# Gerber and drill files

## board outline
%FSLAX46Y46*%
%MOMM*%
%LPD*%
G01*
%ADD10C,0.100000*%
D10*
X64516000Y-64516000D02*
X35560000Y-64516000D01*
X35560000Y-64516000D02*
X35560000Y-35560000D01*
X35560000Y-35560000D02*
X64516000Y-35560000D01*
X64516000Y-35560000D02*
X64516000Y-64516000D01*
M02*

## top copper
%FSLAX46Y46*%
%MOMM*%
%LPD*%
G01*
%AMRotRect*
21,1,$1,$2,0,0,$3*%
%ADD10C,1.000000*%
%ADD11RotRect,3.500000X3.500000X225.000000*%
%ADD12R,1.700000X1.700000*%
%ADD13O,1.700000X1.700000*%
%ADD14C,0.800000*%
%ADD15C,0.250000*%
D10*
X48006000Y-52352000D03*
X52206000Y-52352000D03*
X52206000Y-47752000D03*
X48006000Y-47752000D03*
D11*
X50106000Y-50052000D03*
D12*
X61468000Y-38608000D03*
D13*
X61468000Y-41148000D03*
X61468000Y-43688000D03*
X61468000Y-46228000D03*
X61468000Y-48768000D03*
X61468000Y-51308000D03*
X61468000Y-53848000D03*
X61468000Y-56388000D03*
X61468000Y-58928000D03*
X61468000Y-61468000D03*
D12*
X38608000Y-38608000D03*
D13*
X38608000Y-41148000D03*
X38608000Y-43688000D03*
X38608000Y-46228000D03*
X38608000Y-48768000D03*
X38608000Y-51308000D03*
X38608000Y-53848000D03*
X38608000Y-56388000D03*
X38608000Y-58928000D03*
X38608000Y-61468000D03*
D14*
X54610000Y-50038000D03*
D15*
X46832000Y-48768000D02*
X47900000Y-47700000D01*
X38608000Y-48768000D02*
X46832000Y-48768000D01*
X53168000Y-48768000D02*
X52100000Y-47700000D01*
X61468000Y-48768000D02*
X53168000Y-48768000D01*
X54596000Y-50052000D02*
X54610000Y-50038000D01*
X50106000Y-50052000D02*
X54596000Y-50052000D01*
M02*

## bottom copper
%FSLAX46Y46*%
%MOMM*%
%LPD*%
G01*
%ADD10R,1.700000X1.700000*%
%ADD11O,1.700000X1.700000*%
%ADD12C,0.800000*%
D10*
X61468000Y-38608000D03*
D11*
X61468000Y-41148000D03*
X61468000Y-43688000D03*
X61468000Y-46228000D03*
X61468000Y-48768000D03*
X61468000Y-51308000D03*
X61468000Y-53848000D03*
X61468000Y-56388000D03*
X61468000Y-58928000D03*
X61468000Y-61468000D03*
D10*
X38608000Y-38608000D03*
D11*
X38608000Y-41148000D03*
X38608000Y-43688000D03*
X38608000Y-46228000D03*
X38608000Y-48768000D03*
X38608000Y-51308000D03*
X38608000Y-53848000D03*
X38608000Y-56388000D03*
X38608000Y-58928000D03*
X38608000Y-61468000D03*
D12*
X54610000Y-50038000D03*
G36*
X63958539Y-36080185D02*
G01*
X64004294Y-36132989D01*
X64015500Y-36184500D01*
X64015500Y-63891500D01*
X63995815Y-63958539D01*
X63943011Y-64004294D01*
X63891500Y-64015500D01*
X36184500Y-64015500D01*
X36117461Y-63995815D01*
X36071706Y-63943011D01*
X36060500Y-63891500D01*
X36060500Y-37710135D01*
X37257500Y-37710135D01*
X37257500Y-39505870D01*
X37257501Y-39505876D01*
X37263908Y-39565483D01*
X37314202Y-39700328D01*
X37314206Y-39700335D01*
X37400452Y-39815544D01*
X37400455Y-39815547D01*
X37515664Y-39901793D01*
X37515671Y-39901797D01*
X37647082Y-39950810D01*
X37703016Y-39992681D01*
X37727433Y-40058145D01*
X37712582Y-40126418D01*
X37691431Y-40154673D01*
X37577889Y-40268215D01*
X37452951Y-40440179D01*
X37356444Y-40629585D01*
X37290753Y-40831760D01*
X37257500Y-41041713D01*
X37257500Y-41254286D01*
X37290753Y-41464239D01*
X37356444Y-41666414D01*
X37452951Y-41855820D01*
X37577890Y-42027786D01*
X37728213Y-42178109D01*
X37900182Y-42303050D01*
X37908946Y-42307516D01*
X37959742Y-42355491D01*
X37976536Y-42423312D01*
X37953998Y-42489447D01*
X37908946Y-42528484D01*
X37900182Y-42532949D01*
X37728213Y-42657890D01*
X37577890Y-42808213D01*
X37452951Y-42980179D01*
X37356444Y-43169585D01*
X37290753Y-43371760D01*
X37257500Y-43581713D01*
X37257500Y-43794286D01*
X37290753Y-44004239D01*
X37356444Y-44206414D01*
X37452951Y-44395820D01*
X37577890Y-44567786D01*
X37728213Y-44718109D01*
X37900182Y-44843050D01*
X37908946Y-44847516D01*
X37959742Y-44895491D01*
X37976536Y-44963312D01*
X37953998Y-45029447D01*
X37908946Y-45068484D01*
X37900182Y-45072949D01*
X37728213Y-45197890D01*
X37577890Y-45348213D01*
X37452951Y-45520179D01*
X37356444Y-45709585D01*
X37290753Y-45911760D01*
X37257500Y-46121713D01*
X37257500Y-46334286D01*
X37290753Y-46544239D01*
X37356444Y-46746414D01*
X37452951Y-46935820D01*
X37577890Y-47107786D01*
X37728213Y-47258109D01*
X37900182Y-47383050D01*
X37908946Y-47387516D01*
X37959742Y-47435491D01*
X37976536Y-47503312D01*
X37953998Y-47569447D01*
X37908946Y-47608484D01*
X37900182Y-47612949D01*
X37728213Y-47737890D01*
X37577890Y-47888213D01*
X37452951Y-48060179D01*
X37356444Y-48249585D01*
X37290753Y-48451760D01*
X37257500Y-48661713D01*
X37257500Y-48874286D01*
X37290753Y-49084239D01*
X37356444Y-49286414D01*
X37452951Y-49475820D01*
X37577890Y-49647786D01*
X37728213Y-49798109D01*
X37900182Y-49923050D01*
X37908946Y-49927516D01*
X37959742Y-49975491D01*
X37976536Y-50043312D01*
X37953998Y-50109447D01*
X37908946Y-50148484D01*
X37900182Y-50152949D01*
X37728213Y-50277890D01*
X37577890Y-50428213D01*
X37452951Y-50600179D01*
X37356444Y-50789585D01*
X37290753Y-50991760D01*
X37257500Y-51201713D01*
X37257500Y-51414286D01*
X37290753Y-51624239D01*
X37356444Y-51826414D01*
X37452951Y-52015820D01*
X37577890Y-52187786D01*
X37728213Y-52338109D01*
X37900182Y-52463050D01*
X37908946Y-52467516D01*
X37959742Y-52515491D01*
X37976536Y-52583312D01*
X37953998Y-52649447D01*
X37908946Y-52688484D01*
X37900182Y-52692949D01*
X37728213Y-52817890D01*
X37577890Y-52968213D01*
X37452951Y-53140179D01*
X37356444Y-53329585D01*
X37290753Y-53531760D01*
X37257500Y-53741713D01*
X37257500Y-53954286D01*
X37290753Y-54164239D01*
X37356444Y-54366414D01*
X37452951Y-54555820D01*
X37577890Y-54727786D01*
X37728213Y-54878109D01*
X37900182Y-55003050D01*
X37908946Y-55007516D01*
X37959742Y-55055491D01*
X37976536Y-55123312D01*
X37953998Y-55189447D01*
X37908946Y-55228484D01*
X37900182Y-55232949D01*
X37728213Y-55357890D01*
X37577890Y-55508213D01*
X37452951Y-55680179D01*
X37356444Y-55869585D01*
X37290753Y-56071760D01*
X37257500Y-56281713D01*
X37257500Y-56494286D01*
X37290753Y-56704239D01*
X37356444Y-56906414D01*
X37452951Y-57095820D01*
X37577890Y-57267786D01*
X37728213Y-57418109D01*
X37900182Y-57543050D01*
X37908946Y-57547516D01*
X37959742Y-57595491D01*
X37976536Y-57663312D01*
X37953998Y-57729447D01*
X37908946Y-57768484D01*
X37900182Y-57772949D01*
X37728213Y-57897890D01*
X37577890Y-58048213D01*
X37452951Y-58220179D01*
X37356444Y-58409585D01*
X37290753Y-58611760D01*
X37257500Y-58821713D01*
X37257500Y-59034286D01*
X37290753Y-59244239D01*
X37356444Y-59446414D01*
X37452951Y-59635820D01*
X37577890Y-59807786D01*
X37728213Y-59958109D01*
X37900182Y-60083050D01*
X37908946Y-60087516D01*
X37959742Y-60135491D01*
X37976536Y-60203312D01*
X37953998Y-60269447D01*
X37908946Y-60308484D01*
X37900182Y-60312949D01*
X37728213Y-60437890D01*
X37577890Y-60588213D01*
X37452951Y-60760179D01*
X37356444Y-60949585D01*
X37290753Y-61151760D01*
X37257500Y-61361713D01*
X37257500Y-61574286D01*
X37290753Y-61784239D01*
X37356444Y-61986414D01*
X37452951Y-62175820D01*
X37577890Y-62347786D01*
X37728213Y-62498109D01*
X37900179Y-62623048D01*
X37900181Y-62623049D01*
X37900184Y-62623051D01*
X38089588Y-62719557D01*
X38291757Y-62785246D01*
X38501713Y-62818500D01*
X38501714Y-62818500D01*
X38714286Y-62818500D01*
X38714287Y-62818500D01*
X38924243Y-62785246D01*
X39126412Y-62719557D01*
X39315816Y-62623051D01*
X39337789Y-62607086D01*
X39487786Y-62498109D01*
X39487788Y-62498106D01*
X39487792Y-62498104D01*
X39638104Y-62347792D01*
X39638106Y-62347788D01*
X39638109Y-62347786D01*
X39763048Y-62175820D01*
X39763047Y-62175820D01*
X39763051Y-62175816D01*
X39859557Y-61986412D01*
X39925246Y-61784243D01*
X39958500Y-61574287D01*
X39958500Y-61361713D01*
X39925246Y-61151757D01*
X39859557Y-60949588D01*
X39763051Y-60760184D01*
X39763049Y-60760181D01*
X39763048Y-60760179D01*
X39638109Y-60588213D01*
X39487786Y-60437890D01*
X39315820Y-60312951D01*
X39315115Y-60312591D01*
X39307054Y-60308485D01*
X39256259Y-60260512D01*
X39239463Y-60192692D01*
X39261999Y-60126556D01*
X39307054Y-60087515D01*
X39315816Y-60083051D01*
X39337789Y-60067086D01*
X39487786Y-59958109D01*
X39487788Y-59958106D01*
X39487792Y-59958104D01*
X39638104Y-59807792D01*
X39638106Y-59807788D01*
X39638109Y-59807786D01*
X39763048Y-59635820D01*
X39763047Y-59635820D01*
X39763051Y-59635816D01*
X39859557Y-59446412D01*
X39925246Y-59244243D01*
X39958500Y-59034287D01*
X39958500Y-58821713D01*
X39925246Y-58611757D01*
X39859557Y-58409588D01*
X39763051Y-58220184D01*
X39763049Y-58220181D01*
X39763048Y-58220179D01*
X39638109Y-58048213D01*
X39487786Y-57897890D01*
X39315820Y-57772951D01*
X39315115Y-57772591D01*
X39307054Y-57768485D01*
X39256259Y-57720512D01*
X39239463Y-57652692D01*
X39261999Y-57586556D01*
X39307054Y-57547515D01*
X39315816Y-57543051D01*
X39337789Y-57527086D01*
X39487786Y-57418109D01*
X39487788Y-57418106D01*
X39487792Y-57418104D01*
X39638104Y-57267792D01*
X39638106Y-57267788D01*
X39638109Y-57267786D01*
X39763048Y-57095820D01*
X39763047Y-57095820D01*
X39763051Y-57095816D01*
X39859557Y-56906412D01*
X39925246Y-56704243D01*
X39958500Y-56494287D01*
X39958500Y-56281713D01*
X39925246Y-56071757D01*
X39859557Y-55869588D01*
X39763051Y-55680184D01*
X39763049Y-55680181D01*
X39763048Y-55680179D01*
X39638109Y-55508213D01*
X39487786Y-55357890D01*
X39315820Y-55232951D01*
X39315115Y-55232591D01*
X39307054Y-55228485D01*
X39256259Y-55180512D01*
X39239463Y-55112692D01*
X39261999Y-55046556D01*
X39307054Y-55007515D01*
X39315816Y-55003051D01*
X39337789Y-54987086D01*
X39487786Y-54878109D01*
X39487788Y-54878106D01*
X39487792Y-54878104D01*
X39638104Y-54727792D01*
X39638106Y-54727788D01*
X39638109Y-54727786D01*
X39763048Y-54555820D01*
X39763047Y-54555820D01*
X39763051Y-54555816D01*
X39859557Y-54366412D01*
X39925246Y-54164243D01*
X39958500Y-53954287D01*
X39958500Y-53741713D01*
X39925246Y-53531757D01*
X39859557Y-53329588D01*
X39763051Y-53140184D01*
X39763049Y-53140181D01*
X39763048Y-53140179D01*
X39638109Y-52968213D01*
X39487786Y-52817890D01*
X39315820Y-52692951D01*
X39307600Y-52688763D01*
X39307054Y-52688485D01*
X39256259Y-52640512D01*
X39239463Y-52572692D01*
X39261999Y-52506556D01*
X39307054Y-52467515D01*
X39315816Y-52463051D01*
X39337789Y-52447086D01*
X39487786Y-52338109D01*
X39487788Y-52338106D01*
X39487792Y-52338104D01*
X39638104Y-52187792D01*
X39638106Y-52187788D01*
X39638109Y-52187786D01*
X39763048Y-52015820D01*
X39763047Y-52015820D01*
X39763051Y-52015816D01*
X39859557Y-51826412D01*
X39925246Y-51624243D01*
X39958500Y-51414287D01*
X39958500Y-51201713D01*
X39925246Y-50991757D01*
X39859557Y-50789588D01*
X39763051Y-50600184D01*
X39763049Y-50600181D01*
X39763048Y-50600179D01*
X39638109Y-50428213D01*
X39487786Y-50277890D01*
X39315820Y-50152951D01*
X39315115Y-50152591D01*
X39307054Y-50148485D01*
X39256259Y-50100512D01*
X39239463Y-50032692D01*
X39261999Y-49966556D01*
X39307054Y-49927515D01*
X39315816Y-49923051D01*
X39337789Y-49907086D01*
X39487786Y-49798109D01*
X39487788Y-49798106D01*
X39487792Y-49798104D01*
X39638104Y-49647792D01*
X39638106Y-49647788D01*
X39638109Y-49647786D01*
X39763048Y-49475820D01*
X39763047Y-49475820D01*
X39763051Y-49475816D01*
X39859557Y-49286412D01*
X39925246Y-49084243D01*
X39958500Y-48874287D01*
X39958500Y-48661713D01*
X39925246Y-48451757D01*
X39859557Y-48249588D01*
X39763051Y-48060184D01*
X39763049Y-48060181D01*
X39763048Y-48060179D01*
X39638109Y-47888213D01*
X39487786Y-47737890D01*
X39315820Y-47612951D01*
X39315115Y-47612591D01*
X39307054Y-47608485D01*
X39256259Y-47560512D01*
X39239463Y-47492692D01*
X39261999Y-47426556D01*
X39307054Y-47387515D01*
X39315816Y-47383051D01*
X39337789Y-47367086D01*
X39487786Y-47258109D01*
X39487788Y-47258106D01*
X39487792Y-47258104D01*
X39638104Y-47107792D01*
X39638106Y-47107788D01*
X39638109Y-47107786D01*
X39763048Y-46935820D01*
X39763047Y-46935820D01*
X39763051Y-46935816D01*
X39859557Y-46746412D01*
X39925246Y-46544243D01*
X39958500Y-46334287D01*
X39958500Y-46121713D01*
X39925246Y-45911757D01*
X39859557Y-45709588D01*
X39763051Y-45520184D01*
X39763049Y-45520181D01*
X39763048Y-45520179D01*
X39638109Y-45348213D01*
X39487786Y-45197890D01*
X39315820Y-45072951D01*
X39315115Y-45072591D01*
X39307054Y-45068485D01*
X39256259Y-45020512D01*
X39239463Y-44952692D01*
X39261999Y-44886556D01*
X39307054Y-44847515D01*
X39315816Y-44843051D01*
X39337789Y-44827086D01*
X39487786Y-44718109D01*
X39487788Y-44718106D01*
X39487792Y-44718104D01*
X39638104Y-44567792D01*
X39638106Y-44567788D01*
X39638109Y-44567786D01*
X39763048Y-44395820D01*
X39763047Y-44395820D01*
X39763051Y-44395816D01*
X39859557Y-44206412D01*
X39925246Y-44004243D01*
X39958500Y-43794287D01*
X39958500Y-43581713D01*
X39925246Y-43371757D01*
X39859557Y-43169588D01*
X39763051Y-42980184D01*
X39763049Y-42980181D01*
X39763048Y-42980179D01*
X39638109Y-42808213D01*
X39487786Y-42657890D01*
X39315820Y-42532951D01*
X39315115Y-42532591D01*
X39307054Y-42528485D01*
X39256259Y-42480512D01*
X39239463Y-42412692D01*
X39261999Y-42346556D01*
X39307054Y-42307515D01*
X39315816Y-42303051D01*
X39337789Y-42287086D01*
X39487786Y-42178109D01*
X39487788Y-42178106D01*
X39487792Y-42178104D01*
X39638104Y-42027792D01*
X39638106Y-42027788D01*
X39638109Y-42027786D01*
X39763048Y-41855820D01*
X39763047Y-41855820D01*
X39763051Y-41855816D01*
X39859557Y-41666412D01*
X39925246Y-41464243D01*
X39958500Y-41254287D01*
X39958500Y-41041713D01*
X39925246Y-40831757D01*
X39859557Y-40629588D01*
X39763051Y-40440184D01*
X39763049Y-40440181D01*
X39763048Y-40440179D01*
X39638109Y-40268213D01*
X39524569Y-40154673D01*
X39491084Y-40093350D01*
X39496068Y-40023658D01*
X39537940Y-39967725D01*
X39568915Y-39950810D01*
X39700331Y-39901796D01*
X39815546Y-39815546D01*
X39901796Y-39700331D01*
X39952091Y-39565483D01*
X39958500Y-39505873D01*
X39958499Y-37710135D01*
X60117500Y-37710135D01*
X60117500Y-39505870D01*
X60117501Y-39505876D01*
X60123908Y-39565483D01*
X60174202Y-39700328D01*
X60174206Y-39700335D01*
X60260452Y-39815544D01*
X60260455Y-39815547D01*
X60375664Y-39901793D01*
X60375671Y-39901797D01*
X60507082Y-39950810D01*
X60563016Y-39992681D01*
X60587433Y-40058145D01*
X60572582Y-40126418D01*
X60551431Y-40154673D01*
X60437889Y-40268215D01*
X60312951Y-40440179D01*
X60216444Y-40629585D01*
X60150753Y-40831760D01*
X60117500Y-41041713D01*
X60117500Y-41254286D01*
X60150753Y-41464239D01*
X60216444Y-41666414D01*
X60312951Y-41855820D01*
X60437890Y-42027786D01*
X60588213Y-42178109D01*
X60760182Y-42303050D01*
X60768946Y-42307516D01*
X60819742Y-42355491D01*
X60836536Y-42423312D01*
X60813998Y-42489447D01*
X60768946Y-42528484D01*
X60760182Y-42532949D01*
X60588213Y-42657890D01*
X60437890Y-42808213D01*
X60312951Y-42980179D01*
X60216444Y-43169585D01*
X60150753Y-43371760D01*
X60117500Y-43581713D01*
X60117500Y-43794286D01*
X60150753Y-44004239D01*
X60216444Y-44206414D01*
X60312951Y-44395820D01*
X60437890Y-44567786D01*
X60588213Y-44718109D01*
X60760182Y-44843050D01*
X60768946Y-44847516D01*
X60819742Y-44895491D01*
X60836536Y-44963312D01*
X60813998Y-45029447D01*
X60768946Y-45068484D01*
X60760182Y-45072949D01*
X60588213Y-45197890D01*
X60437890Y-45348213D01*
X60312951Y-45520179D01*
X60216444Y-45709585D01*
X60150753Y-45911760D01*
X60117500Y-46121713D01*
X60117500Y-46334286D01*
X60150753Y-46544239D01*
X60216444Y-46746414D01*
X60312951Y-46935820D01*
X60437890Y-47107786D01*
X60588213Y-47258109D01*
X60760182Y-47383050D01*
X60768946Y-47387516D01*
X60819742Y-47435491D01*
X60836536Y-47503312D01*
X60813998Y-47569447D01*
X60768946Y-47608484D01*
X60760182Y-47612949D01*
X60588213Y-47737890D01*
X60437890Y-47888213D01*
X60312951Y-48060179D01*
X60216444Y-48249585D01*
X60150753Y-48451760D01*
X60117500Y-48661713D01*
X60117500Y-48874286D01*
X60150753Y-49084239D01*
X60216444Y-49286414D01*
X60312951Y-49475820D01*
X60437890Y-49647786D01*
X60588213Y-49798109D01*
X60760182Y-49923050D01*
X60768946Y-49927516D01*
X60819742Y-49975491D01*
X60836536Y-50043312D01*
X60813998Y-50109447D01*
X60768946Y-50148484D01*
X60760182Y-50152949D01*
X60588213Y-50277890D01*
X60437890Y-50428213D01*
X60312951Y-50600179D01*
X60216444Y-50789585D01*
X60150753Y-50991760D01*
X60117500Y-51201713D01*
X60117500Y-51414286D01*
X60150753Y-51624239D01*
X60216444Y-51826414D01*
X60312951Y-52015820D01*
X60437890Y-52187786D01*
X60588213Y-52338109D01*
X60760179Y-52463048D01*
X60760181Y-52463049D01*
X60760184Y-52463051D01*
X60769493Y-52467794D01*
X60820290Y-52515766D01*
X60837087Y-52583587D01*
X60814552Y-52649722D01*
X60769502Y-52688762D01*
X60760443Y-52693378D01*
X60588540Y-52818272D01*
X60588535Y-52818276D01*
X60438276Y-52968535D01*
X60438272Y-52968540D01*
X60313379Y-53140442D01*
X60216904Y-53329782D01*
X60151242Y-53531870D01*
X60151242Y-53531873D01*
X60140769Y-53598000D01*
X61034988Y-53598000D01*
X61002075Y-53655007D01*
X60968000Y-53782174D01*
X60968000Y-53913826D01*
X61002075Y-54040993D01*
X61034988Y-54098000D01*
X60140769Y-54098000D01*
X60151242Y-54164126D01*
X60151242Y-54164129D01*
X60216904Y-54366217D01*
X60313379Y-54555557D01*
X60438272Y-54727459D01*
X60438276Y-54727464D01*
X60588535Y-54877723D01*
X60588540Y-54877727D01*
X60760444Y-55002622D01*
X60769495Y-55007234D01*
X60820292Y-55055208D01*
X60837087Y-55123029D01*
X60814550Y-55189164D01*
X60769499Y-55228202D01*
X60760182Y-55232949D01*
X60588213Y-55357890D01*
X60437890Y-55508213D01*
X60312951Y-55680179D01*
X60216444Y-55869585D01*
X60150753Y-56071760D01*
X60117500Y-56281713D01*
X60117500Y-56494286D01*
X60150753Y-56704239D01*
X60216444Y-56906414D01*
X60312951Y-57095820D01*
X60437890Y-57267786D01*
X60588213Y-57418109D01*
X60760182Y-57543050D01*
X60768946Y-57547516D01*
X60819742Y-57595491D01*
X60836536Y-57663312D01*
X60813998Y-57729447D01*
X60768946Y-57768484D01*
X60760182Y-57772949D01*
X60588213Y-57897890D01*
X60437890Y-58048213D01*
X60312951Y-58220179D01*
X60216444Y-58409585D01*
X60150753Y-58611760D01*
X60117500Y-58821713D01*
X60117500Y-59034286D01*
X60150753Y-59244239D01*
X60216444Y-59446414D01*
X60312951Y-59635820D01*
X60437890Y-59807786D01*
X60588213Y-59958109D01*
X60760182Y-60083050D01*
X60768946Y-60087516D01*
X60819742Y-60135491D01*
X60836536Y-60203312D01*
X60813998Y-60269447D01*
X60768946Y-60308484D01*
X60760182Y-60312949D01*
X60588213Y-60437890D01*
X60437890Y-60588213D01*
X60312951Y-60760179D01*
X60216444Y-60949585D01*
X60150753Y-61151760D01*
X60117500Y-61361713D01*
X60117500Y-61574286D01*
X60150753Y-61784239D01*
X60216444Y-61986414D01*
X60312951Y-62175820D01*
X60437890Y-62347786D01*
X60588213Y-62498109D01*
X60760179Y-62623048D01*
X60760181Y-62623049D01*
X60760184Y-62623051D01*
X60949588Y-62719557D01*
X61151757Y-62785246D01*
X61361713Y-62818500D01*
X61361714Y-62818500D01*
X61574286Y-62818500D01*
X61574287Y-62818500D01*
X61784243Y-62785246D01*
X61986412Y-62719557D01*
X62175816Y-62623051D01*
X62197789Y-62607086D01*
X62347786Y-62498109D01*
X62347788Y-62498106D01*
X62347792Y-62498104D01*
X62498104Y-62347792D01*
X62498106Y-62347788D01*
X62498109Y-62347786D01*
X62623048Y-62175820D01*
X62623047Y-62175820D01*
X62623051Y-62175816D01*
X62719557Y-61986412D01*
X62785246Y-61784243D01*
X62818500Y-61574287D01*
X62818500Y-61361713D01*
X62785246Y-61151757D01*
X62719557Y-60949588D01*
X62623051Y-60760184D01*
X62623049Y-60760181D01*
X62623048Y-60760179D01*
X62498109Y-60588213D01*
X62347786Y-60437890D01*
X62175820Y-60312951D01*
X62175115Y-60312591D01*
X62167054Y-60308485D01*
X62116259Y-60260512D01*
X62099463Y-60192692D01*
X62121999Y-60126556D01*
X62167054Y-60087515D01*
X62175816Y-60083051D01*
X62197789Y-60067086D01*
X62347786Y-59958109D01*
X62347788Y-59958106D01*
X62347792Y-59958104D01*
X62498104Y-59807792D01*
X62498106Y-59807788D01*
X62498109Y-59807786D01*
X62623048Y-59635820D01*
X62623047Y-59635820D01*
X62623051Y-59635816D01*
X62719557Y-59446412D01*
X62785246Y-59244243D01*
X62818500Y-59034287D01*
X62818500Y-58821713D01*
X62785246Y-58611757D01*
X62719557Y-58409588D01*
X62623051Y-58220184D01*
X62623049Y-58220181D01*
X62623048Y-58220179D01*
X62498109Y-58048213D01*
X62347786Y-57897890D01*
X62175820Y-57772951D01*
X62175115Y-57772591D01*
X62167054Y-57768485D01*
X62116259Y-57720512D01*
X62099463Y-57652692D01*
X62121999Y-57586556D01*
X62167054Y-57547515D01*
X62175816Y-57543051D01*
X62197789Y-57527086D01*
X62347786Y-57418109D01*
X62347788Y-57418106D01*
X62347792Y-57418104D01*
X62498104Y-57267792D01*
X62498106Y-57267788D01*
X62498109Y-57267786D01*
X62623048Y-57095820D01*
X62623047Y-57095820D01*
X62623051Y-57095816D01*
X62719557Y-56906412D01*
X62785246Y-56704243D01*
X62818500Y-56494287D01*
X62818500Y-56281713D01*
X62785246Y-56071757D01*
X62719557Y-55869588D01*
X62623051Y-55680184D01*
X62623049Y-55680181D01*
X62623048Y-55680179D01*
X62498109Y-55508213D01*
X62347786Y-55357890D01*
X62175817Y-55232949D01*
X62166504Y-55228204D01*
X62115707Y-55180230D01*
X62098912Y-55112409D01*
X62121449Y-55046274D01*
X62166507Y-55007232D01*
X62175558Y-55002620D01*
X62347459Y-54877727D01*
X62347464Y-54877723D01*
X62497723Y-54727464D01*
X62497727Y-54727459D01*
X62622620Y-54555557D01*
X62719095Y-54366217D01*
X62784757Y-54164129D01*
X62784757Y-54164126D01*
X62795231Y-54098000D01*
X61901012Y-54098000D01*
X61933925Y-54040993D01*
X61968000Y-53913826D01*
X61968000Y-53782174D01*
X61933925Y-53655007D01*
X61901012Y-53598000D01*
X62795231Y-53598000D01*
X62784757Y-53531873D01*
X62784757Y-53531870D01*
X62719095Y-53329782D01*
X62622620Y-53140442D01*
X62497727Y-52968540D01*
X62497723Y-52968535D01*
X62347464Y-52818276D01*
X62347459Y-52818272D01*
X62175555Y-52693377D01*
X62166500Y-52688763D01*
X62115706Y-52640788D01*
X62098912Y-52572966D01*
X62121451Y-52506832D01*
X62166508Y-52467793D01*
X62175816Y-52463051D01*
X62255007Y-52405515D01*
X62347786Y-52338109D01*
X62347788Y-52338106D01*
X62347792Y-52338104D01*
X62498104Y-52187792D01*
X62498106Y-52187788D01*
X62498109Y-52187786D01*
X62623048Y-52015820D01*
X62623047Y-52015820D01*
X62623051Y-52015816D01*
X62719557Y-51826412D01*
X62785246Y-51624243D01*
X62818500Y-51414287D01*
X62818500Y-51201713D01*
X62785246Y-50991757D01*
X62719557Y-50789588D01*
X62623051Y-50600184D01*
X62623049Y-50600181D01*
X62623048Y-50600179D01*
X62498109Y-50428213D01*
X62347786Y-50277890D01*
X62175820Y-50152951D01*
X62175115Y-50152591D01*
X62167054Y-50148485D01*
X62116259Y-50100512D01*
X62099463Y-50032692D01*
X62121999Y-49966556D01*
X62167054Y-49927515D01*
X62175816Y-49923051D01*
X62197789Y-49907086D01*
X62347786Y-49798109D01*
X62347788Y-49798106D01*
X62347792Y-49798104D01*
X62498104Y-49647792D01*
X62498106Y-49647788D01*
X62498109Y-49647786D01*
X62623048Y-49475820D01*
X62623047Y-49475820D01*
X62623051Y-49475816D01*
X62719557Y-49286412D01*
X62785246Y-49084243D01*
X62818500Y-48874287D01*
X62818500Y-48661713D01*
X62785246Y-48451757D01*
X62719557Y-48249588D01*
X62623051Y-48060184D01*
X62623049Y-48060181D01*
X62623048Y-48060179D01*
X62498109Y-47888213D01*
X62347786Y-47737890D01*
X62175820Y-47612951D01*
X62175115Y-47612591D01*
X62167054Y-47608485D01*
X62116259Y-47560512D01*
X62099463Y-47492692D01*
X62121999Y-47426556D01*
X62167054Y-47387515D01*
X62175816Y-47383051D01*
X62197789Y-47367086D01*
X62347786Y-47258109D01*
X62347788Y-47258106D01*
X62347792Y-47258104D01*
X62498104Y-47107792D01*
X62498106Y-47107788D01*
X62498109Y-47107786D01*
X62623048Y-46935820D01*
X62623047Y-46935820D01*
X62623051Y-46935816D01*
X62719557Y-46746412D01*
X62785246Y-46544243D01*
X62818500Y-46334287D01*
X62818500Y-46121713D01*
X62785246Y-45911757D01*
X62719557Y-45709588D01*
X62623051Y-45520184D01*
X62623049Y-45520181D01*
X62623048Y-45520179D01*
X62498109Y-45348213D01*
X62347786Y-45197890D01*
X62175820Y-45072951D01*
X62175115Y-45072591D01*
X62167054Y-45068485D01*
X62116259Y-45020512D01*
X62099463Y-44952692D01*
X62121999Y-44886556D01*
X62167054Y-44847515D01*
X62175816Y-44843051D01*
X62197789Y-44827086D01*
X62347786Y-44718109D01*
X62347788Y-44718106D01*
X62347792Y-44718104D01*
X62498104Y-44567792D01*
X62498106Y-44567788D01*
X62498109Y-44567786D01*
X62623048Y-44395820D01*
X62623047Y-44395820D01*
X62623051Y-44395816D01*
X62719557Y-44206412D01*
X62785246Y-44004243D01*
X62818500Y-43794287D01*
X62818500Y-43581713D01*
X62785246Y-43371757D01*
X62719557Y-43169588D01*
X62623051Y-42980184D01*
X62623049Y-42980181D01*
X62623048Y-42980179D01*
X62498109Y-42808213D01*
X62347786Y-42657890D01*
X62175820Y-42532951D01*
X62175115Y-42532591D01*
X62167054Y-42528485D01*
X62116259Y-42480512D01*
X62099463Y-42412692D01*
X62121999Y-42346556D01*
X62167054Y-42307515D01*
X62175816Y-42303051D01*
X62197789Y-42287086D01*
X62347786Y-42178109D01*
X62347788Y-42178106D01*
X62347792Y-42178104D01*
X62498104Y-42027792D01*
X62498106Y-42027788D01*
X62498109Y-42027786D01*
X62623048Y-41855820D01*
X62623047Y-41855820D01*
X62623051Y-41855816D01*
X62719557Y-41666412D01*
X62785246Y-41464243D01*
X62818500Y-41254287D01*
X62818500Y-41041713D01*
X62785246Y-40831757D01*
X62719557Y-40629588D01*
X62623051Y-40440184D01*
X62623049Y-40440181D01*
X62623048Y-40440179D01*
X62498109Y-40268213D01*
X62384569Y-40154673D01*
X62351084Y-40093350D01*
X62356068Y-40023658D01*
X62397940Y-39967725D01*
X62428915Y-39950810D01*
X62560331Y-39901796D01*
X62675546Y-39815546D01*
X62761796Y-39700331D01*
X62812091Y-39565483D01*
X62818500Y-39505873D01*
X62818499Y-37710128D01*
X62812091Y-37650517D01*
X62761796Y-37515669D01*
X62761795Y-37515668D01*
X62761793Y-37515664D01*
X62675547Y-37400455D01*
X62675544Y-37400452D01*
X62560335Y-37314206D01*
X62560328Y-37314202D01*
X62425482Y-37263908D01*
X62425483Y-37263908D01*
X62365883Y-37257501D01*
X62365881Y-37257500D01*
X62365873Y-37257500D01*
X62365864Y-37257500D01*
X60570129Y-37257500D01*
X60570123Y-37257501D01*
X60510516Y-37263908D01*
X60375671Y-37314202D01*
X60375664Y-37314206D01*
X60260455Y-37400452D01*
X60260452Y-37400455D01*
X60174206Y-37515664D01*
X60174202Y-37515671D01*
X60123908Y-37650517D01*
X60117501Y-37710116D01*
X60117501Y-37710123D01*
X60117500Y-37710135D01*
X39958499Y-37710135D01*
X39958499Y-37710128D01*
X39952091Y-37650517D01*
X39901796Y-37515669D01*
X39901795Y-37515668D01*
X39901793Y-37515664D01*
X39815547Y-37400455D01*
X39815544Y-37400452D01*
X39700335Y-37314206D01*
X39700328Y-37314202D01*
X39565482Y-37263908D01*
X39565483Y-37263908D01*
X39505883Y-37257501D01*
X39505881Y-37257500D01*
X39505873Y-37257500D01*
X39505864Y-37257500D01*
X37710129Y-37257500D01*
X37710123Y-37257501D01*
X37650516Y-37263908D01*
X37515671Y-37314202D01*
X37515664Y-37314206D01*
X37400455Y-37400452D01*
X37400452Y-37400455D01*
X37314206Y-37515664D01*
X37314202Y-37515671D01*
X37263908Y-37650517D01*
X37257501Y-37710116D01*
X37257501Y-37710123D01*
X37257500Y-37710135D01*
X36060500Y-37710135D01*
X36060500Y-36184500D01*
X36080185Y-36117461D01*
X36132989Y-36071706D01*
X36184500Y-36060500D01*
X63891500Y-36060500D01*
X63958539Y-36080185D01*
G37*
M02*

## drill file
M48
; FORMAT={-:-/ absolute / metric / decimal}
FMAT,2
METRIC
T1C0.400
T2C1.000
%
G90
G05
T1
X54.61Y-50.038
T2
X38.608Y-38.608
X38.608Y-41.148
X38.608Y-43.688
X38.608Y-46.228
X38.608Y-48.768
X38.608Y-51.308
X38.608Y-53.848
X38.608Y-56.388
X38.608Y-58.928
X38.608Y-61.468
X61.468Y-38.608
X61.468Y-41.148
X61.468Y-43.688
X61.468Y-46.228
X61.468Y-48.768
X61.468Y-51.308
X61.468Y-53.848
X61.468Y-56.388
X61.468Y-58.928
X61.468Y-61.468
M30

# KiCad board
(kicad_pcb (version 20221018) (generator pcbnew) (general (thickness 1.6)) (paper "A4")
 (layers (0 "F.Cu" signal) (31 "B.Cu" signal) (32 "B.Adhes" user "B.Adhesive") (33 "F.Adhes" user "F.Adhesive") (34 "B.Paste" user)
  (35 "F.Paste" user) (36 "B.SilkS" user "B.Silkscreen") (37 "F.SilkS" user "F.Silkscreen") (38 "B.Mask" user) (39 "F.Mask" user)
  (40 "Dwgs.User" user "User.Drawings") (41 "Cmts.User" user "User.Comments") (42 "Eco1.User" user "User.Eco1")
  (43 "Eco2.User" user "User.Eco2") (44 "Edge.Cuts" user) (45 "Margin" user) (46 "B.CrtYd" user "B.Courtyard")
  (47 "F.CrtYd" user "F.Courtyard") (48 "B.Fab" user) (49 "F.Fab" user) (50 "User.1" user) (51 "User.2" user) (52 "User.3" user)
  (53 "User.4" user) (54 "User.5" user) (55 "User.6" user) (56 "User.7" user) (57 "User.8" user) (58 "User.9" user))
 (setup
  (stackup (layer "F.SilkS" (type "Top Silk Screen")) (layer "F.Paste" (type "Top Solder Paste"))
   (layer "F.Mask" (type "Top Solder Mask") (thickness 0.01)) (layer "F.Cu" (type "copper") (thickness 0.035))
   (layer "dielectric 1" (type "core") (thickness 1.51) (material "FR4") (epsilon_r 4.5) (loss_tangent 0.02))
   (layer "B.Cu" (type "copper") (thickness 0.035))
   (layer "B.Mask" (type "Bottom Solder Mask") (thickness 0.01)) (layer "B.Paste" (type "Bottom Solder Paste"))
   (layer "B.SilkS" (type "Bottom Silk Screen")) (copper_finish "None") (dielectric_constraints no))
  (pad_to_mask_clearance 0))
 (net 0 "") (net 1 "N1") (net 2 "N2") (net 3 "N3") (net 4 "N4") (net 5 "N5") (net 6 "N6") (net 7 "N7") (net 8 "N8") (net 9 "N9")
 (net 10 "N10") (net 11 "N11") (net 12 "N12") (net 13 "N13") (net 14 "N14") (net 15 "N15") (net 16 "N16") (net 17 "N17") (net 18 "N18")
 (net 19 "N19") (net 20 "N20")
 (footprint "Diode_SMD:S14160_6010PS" (layer "F.Cu") (at 50.106 50.052 180)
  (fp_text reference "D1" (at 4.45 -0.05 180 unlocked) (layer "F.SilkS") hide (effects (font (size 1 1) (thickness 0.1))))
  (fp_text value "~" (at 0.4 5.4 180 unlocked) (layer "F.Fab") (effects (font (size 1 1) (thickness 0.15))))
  (fp_rect (start 0 1.75) (end 0 1.75) (stroke (width 0.1) (type solid)) (fill none) (layer "F.Cu"))
  (pad "1" smd circle (at 2.1 -2.3 180) (size 1 1) (layers "F.Cu" "F.Paste" "F.Mask"))
  (pad "2" smd circle (at -2.1 -2.3 180) (size 1 1) (layers "F.Cu" "F.Paste" "F.Mask"))
  (pad "3" smd circle (at -2.1 2.3 180) (size 1 1) (layers "F.Cu" "F.Paste" "F.Mask") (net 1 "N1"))
  (pad "4" smd circle (at 2.1 2.3 180) (size 1 1) (layers "F.Cu" "F.Paste" "F.Mask") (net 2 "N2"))
  (pad "5" smd rect (at 0 0 225) (size 3.5 3.5) (layers "F.Cu" "F.Paste" "F.Mask") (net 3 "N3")))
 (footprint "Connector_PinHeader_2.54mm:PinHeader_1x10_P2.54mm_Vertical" (layer "B.Cu") (at 61.468 38.608 180)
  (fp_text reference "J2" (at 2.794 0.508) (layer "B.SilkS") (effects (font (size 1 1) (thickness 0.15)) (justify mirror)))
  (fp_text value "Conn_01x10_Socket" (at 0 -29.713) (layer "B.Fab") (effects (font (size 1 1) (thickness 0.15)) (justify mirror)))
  (pad "1" thru_hole rect (at 0 0 180) (size 1.7 1.7) (drill 1) (layers "*.Cu" "*.Mask") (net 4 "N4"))
  (pad "2" thru_hole oval (at 0 -2.54 180) (size 1.7 1.7) (drill 1) (layers "*.Cu" "*.Mask") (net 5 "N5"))
  (pad "3" thru_hole oval (at 0 -5.08 180) (size 1.7 1.7) (drill 1) (layers "*.Cu" "*.Mask") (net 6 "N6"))
  (pad "4" thru_hole oval (at 0 -7.62 180) (size 1.7 1.7) (drill 1) (layers "*.Cu" "*.Mask") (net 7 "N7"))
  (pad "5" thru_hole oval (at 0 -10.16 180) (size 1.7 1.7) (drill 1) (layers "*.Cu" "*.Mask") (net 1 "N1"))
  (pad "6" thru_hole oval (at 0 -12.7 180) (size 1.7 1.7) (drill 1) (layers "*.Cu" "*.Mask") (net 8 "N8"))
  (pad "7" thru_hole oval (at 0 -15.24 180) (size 1.7 1.7) (drill 1) (layers "*.Cu" "*.Mask") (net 3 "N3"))
  (pad "8" thru_hole oval (at 0 -17.78 180) (size 1.7 1.7) (drill 1) (layers "*.Cu" "*.Mask") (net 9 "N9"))
  (pad "9" thru_hole oval (at 0 -20.32 180) (size 1.7 1.7) (drill 1) (layers "*.Cu" "*.Mask") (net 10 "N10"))
  (pad "10" thru_hole oval (at 0 -22.86 180) (size 1.7 1.7) (drill 1) (layers "*.Cu" "*.Mask") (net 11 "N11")))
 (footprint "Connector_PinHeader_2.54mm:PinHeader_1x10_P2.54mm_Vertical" (layer "B.Cu") (at 38.608 38.608 180)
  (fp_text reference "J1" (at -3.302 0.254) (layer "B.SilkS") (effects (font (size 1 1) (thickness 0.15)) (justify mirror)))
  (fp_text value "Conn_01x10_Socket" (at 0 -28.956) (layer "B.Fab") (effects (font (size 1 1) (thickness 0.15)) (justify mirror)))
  (pad "1" thru_hole rect (at 0 0 180) (size 1.7 1.7) (drill 1) (layers "*.Cu" "*.Mask") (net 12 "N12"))
  (pad "2" thru_hole oval (at 0 -2.54 180) (size 1.7 1.7) (drill 1) (layers "*.Cu" "*.Mask") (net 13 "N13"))
  (pad "3" thru_hole oval (at 0 -5.08 180) (size 1.7 1.7) (drill 1) (layers "*.Cu" "*.Mask") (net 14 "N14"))
  (pad "4" thru_hole oval (at 0 -7.62 180) (size 1.7 1.7) (drill 1) (layers "*.Cu" "*.Mask") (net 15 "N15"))
  (pad "5" thru_hole oval (at 0 -10.16 180) (size 1.7 1.7) (drill 1) (layers "*.Cu" "*.Mask") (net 2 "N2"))
  (pad "6" thru_hole oval (at 0 -12.7 180) (size 1.7 1.7) (drill 1) (layers "*.Cu" "*.Mask") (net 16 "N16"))
  (pad "7" thru_hole oval (at 0 -15.24 180) (size 1.7 1.7) (drill 1) (layers "*.Cu" "*.Mask") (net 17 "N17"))
  (pad "8" thru_hole oval (at 0 -17.78 180) (size 1.7 1.7) (drill 1) (layers "*.Cu" "*.Mask") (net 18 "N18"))
  (pad "9" thru_hole oval (at 0 -20.32 180) (size 1.7 1.7) (drill 1) (layers "*.Cu" "*.Mask") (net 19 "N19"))
  (pad "10" thru_hole oval (at 0 -22.86 180) (size 1.7 1.7) (drill 1) (layers "*.Cu" "*.Mask") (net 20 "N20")))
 (gr_line (start 64.516 64.516) (end 35.56 64.516) (stroke (width 0.1) (type default)) (layer "Edge.Cuts"))
 (gr_line (start 35.56 64.516) (end 35.56 35.56) (stroke (width 0.1) (type default)) (layer "Edge.Cuts"))
 (gr_line (start 35.56 35.56) (end 64.516 35.56) (stroke (width 0.1) (type default)) (layer "Edge.Cuts"))
 (gr_line (start 64.516 35.56) (end 64.516 64.516) (stroke (width 0.1) (type default)) (layer "Edge.Cuts"))
 (segment (start 46.832 48.768) (end 47.9 47.7) (width 0.25) (layer "F.Cu") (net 2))
 (segment (start 38.608 48.768) (end 46.832 48.768) (width 0.25) (layer "F.Cu") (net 2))
 (segment (start 53.168 48.768) (end 52.1 47.7) (width 0.25) (layer "F.Cu") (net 1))
 (segment (start 61.468 48.768) (end 53.168 48.768) (width 0.25) (layer "F.Cu") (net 1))
 (segment (start 54.596 50.052) (end 54.61 50.038) (width 0.25) (layer "F.Cu") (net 3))
 (segment (start 50.106 50.052) (end 54.596 50.052) (width 0.25) (layer "F.Cu") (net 3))
 (via (at 54.61 50.038) (size 0.8) (drill 0.4) (layers "F.Cu" "B.Cu") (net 3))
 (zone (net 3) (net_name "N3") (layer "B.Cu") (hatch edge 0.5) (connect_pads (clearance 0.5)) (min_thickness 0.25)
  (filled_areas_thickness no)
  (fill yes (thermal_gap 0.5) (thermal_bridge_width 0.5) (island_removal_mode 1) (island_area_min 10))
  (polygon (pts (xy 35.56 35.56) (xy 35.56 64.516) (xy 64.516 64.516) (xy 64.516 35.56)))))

